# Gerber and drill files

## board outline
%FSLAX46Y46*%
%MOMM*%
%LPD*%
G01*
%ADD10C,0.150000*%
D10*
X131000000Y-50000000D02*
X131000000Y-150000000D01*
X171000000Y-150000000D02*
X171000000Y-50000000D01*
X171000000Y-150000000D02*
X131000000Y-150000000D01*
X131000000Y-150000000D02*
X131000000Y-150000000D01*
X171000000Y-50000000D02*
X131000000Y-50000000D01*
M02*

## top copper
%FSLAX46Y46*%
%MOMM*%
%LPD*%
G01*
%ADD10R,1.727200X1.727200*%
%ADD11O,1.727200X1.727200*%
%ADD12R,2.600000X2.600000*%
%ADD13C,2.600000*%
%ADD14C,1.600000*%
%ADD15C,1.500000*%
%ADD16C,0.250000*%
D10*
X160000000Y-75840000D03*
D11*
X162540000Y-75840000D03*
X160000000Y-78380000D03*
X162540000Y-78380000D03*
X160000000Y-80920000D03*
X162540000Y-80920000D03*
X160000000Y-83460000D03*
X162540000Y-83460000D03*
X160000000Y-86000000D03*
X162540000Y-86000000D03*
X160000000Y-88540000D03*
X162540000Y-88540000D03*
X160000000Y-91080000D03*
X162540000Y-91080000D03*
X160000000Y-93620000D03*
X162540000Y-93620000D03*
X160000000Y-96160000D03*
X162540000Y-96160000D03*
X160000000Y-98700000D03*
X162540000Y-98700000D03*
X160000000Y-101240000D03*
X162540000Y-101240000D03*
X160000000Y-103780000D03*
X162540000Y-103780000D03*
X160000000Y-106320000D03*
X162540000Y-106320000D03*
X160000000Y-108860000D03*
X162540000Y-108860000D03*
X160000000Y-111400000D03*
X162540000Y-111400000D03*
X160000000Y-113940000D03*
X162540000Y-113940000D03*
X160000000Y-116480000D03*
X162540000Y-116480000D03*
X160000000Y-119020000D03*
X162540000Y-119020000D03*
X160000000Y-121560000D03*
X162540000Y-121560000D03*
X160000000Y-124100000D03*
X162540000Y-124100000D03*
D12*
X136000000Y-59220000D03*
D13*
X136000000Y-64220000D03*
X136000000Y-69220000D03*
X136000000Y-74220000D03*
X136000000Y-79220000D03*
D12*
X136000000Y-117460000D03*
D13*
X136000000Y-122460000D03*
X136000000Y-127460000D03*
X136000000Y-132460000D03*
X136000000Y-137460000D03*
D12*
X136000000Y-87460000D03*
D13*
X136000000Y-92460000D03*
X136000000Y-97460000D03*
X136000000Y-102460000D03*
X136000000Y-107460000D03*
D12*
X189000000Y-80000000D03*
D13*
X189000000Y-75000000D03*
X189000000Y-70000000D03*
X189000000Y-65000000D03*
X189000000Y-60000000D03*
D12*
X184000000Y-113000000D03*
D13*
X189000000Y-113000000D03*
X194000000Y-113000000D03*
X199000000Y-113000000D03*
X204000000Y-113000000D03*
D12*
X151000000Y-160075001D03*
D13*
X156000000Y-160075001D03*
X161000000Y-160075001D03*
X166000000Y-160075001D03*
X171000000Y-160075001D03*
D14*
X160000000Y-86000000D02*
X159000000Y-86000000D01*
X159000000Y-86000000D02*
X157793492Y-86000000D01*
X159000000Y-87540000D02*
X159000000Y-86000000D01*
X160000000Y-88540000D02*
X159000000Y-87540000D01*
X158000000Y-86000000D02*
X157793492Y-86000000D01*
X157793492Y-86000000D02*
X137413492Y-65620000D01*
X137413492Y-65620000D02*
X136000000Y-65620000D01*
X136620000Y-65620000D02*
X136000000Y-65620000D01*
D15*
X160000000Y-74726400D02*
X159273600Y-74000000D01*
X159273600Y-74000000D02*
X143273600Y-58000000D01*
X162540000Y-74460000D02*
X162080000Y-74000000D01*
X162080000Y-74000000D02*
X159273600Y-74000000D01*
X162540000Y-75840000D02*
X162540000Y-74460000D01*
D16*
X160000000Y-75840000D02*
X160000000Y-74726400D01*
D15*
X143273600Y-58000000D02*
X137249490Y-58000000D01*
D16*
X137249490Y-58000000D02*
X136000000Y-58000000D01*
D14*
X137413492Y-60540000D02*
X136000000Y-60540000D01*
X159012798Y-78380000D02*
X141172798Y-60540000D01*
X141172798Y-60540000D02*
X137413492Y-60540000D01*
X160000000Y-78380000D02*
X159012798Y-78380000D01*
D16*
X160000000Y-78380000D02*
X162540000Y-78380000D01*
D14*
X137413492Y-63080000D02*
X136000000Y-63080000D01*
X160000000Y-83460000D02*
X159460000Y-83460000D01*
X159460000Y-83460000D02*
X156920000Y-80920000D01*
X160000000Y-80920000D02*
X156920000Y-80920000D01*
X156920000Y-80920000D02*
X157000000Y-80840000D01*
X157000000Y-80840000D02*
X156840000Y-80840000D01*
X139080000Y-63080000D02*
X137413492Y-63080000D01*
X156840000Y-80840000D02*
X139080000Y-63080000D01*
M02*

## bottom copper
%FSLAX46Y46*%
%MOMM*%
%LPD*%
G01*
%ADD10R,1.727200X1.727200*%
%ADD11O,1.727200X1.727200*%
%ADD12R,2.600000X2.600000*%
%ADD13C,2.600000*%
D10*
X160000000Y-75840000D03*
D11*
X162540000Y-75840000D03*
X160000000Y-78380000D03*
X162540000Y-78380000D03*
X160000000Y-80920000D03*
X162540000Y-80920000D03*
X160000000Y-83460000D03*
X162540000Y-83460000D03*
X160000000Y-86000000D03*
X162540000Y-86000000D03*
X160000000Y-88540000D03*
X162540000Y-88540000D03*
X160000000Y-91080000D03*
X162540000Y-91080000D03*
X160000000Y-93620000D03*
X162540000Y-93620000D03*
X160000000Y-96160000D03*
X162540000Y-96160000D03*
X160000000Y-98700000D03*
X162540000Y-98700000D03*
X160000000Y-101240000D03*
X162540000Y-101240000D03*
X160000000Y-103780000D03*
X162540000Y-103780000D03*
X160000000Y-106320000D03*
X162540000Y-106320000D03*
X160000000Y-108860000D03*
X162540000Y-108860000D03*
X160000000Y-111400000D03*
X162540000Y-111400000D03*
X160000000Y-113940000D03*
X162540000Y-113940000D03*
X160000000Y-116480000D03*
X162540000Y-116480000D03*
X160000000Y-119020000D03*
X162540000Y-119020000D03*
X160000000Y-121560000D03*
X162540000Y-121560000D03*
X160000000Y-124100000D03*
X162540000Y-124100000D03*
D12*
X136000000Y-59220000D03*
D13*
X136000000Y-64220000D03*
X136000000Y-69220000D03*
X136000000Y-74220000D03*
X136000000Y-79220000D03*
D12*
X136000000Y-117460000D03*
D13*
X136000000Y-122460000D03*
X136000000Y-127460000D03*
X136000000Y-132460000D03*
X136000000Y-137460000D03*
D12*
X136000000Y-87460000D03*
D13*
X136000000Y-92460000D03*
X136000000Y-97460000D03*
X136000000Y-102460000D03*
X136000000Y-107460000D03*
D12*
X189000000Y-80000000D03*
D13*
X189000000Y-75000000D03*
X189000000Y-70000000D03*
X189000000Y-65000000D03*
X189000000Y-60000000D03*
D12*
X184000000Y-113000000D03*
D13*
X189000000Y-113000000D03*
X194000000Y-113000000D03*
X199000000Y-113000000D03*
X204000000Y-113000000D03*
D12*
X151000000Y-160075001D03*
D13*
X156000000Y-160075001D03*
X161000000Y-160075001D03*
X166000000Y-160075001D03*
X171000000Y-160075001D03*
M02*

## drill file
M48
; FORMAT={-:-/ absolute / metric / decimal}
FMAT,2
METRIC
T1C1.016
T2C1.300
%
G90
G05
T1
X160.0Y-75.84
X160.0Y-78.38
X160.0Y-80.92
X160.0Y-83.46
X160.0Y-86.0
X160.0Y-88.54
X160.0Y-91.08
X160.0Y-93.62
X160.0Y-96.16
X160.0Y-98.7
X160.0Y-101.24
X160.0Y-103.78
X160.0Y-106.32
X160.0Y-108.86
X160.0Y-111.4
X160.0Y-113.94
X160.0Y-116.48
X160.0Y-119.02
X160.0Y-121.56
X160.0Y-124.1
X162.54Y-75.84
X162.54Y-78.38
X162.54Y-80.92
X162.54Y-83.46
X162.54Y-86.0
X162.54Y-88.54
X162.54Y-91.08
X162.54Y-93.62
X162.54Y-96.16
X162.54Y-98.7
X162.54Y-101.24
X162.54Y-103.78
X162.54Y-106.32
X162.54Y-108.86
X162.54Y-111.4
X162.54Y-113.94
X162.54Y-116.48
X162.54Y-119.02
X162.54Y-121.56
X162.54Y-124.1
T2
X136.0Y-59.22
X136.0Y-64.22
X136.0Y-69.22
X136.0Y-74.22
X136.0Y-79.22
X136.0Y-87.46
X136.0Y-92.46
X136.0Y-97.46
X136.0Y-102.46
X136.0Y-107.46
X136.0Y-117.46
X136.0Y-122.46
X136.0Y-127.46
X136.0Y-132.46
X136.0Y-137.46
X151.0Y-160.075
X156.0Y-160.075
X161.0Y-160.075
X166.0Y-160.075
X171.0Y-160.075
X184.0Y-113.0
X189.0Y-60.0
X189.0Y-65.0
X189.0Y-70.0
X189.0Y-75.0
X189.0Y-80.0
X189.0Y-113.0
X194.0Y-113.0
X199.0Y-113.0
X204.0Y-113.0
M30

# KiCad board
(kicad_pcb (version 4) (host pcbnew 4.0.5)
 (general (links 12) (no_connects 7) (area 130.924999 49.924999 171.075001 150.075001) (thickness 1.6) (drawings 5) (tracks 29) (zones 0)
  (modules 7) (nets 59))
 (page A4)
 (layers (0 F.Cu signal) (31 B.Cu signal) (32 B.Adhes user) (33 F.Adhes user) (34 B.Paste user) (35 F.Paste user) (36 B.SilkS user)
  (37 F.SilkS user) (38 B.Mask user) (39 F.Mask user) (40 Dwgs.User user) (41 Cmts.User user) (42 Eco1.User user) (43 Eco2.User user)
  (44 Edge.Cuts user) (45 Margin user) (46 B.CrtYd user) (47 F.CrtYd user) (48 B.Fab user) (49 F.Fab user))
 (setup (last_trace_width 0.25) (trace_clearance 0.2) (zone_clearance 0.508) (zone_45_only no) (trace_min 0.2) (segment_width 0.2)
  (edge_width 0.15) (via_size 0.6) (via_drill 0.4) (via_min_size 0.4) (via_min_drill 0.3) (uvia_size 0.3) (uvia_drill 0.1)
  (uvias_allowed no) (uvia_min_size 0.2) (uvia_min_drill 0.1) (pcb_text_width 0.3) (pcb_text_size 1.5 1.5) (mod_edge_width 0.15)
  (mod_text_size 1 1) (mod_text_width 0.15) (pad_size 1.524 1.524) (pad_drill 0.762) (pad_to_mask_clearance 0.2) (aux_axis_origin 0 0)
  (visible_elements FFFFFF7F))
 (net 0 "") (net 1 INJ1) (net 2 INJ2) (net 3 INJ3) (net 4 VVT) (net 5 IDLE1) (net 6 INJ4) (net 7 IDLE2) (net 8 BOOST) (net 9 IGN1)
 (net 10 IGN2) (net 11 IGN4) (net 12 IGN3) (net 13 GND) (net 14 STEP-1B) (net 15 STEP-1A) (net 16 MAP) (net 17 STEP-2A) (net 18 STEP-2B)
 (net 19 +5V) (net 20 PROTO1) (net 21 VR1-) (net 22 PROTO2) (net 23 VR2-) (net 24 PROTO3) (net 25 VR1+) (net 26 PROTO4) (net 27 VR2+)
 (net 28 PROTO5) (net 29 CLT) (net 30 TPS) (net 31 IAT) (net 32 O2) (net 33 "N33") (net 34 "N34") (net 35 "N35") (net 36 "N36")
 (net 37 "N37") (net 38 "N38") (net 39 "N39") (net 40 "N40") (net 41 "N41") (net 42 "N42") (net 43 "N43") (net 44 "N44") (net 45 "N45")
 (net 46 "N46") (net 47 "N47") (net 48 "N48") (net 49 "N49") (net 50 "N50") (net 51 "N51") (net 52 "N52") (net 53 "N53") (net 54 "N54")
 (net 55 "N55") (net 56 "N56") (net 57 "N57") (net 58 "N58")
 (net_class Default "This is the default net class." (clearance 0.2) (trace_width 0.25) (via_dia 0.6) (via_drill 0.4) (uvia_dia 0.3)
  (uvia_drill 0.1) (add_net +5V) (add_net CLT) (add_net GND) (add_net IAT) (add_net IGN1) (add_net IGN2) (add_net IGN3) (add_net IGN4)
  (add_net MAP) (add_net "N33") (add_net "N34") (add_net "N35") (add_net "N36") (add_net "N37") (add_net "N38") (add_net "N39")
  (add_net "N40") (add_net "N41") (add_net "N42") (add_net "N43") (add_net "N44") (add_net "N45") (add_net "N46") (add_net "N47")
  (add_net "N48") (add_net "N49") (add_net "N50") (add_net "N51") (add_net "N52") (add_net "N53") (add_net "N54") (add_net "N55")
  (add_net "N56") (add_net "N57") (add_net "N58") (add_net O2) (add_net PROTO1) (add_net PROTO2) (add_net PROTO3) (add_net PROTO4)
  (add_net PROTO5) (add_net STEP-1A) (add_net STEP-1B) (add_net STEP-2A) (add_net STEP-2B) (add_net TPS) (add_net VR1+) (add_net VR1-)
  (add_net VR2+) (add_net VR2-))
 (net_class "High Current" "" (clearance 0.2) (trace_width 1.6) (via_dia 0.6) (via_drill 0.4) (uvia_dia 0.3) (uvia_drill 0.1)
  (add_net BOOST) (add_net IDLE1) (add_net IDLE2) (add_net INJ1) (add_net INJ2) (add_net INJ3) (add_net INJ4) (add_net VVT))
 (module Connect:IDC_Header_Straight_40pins (layer F.Cu) (at 160 75.84 270)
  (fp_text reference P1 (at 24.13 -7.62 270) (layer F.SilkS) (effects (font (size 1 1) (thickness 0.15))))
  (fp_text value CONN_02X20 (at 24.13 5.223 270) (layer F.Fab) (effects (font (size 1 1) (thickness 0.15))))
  (pad 1 thru_hole rect (at 0 0 270) (size 1.7272 1.7272) (drill 1.016) (layers *.Cu *.Mask) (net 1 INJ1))
  (pad 2 thru_hole oval (at 0 -2.54 270) (size 1.7272 1.7272) (drill 1.016) (layers *.Cu *.Mask) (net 1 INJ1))
  (pad 3 thru_hole oval (at 2.54 0 270) (size 1.7272 1.7272) (drill 1.016) (layers *.Cu *.Mask) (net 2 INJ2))
  (pad 4 thru_hole oval (at 2.54 -2.54 270) (size 1.7272 1.7272) (drill 1.016) (layers *.Cu *.Mask) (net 2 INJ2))
  (pad 5 thru_hole oval (at 5.08 0 270) (size 1.7272 1.7272) (drill 1.016) (layers *.Cu *.Mask) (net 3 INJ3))
  (pad 6 thru_hole oval (at 5.08 -2.54 270) (size 1.7272 1.7272) (drill 1.016) (layers *.Cu *.Mask) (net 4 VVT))
  (pad 7 thru_hole oval (at 7.62 0 270) (size 1.7272 1.7272) (drill 1.016) (layers *.Cu *.Mask) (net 3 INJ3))
  (pad 8 thru_hole oval (at 7.62 -2.54 270) (size 1.7272 1.7272) (drill 1.016) (layers *.Cu *.Mask) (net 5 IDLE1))
  (pad 9 thru_hole oval (at 10.16 0 270) (size 1.7272 1.7272) (drill 1.016) (layers *.Cu *.Mask) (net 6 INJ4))
  (pad 10 thru_hole oval (at 10.16 -2.54 270) (size 1.7272 1.7272) (drill 1.016) (layers *.Cu *.Mask) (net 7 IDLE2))
  (pad 11 thru_hole oval (at 12.7 0 270) (size 1.7272 1.7272) (drill 1.016) (layers *.Cu *.Mask) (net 6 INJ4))
  (pad 12 thru_hole oval (at 12.7 -2.54 270) (size 1.7272 1.7272) (drill 1.016) (layers *.Cu *.Mask) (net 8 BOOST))
  (pad 13 thru_hole oval (at 15.24 0 270) (size 1.7272 1.7272) (drill 1.016) (layers *.Cu *.Mask) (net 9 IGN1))
  (pad 14 thru_hole oval (at 15.24 -2.54 270) (size 1.7272 1.7272) (drill 1.016) (layers *.Cu *.Mask) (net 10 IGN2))
  (pad 15 thru_hole oval (at 17.78 0 270) (size 1.7272 1.7272) (drill 1.016) (layers *.Cu *.Mask) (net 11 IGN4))
  (pad 16 thru_hole oval (at 17.78 -2.54 270) (size 1.7272 1.7272) (drill 1.016) (layers *.Cu *.Mask) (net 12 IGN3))
  (pad 17 thru_hole oval (at 20.32 0 270) (size 1.7272 1.7272) (drill 1.016) (layers *.Cu *.Mask) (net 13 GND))
  (pad 18 thru_hole oval (at 20.32 -2.54 270) (size 1.7272 1.7272) (drill 1.016) (layers *.Cu *.Mask) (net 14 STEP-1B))
  (pad 19 thru_hole oval (at 22.86 0 270) (size 1.7272 1.7272) (drill 1.016) (layers *.Cu *.Mask) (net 13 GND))
  (pad 20 thru_hole oval (at 22.86 -2.54 270) (size 1.7272 1.7272) (drill 1.016) (layers *.Cu *.Mask) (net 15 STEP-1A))
  (pad 21 thru_hole oval (at 25.4 0 270) (size 1.7272 1.7272) (drill 1.016) (layers *.Cu *.Mask) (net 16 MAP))
  (pad 22 thru_hole oval (at 25.4 -2.54 270) (size 1.7272 1.7272) (drill 1.016) (layers *.Cu *.Mask) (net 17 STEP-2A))
  (pad 23 thru_hole oval (at 27.94 0 270) (size 1.7272 1.7272) (drill 1.016) (layers *.Cu *.Mask) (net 13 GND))
  (pad 24 thru_hole oval (at 27.94 -2.54 270) (size 1.7272 1.7272) (drill 1.016) (layers *.Cu *.Mask) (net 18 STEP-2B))
  (pad 25 thru_hole oval (at 30.48 0 270) (size 1.7272 1.7272) (drill 1.016) (layers *.Cu *.Mask) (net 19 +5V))
  (pad 26 thru_hole oval (at 30.48 -2.54 270) (size 1.7272 1.7272) (drill 1.016) (layers *.Cu *.Mask) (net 19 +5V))
  (pad 27 thru_hole oval (at 33.02 0 270) (size 1.7272 1.7272) (drill 1.016) (layers *.Cu *.Mask) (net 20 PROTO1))
  (pad 28 thru_hole oval (at 33.02 -2.54 270) (size 1.7272 1.7272) (drill 1.016) (layers *.Cu *.Mask) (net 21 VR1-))
  (pad 29 thru_hole oval (at 35.56 0 270) (size 1.7272 1.7272) (drill 1.016) (layers *.Cu *.Mask) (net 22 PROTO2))
  (pad 30 thru_hole oval (at 35.56 -2.54 270) (size 1.7272 1.7272) (drill 1.016) (layers *.Cu *.Mask) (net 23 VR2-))
  (pad 31 thru_hole oval (at 38.1 0 270) (size 1.7272 1.7272) (drill 1.016) (layers *.Cu *.Mask) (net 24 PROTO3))
  (pad 32 thru_hole oval (at 38.1 -2.54 270) (size 1.7272 1.7272) (drill 1.016) (layers *.Cu *.Mask) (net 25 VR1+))
  (pad 33 thru_hole oval (at 40.64 0 270) (size 1.7272 1.7272) (drill 1.016) (layers *.Cu *.Mask) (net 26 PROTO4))
  (pad 34 thru_hole oval (at 40.64 -2.54 270) (size 1.7272 1.7272) (drill 1.016) (layers *.Cu *.Mask) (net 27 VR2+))
  (pad 35 thru_hole oval (at 43.18 0 270) (size 1.7272 1.7272) (drill 1.016) (layers *.Cu *.Mask) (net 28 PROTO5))
  (pad 36 thru_hole oval (at 43.18 -2.54 270) (size 1.7272 1.7272) (drill 1.016) (layers *.Cu *.Mask) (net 13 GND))
  (pad 37 thru_hole oval (at 45.72 0 270) (size 1.7272 1.7272) (drill 1.016) (layers *.Cu *.Mask) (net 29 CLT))
  (pad 38 thru_hole oval (at 45.72 -2.54 270) (size 1.7272 1.7272) (drill 1.016) (layers *.Cu *.Mask) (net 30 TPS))
  (pad 39 thru_hole oval (at 48.26 0 270) (size 1.7272 1.7272) (drill 1.016) (layers *.Cu *.Mask) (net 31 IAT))
  (pad 40 thru_hole oval (at 48.26 -2.54 270) (size 1.7272 1.7272) (drill 1.016) (layers *.Cu *.Mask) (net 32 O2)))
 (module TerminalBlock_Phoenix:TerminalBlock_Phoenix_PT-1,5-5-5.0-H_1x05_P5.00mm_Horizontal (layer F.Cu) (at 136 59.22 270)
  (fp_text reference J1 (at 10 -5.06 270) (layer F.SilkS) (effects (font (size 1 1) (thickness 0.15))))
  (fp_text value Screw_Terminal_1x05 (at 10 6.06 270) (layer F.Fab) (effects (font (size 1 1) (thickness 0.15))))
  (pad 1 thru_hole rect (at 0 0 270) (size 2.6 2.6) (drill 1.3) (layers *.Cu *.Mask) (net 1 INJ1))
  (pad 2 thru_hole circle (at 5 0 270) (size 2.6 2.6) (drill 1.3) (layers *.Cu *.Mask) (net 2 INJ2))
  (pad 3 thru_hole circle (at 10 0 270) (size 2.6 2.6) (drill 1.3) (layers *.Cu *.Mask) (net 3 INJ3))
  (pad 4 thru_hole circle (at 15 0 270) (size 2.6 2.6) (drill 1.3) (layers *.Cu *.Mask) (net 6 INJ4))
  (pad 5 thru_hole circle (at 20 0 270) (size 2.6 2.6) (drill 1.3) (layers *.Cu *.Mask) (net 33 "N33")))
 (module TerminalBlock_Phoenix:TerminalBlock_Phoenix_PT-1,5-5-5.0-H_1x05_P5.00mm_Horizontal (layer F.Cu) (at 136 117.46 270)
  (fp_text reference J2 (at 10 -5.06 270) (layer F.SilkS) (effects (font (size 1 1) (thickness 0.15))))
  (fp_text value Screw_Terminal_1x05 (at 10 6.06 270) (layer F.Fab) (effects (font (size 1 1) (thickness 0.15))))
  (pad 1 thru_hole rect (at 0 0 270) (size 2.6 2.6) (drill 1.3) (layers *.Cu *.Mask) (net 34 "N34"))
  (pad 2 thru_hole circle (at 5 0 270) (size 2.6 2.6) (drill 1.3) (layers *.Cu *.Mask) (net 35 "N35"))
  (pad 3 thru_hole circle (at 10 0 270) (size 2.6 2.6) (drill 1.3) (layers *.Cu *.Mask) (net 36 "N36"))
  (pad 4 thru_hole circle (at 15 0 270) (size 2.6 2.6) (drill 1.3) (layers *.Cu *.Mask) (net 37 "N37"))
  (pad 5 thru_hole circle (at 20 0 270) (size 2.6 2.6) (drill 1.3) (layers *.Cu *.Mask) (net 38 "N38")))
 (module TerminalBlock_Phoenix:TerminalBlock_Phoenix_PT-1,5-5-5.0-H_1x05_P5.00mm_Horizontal (layer F.Cu) (at 136 87.46 270)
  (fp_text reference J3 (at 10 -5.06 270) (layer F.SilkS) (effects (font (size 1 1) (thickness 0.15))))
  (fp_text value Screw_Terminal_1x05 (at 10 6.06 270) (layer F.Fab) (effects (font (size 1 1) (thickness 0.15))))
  (pad 1 thru_hole rect (at 0 0 270) (size 2.6 2.6) (drill 1.3) (layers *.Cu *.Mask) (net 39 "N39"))
  (pad 2 thru_hole circle (at 5 0 270) (size 2.6 2.6) (drill 1.3) (layers *.Cu *.Mask) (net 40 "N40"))
  (pad 3 thru_hole circle (at 10 0 270) (size 2.6 2.6) (drill 1.3) (layers *.Cu *.Mask) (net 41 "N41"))
  (pad 4 thru_hole circle (at 15 0 270) (size 2.6 2.6) (drill 1.3) (layers *.Cu *.Mask) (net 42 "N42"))
  (pad 5 thru_hole circle (at 20 0 270) (size 2.6 2.6) (drill 1.3) (layers *.Cu *.Mask) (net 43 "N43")))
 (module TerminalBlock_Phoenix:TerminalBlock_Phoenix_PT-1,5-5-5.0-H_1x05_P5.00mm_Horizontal (layer F.Cu) (at 189 80 90)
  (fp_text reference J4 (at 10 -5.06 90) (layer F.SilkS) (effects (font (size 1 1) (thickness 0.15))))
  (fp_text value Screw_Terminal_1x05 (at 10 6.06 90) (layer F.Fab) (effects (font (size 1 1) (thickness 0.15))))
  (pad 1 thru_hole rect (at 0 0 90) (size 2.6 2.6) (drill 1.3) (layers *.Cu *.Mask) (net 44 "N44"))
  (pad 2 thru_hole circle (at 5 0 90) (size 2.6 2.6) (drill 1.3) (layers *.Cu *.Mask) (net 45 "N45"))
  (pad 3 thru_hole circle (at 10 0 90) (size 2.6 2.6) (drill 1.3) (layers *.Cu *.Mask) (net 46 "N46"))
  (pad 4 thru_hole circle (at 15 0 90) (size 2.6 2.6) (drill 1.3) (layers *.Cu *.Mask) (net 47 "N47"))
  (pad 5 thru_hole circle (at 20 0 90) (size 2.6 2.6) (drill 1.3) (layers *.Cu *.Mask) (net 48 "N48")))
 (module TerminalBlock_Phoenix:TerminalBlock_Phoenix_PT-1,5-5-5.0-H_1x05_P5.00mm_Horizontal (layer F.Cu) (at 184 113)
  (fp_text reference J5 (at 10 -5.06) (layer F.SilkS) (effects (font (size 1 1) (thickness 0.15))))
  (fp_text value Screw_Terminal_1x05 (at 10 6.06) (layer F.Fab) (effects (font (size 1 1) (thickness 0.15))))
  (pad 1 thru_hole rect (at 0 0) (size 2.6 2.6) (drill 1.3) (layers *.Cu *.Mask) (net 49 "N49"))
  (pad 2 thru_hole circle (at 5 0) (size 2.6 2.6) (drill 1.3) (layers *.Cu *.Mask) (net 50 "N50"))
  (pad 3 thru_hole circle (at 10 0) (size 2.6 2.6) (drill 1.3) (layers *.Cu *.Mask) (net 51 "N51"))
  (pad 4 thru_hole circle (at 15 0) (size 2.6 2.6) (drill 1.3) (layers *.Cu *.Mask) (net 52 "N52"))
  (pad 5 thru_hole circle (at 20 0) (size 2.6 2.6) (drill 1.3) (layers *.Cu *.Mask) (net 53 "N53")))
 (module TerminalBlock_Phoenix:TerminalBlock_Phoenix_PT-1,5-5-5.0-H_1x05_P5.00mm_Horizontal (layer F.Cu) (at 151 160.075001)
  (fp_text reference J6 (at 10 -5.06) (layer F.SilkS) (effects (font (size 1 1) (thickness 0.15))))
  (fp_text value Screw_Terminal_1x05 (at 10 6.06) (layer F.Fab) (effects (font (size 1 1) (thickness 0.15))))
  (pad 1 thru_hole rect (at 0 0) (size 2.6 2.6) (drill 1.3) (layers *.Cu *.Mask) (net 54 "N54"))
  (pad 2 thru_hole circle (at 5 0) (size 2.6 2.6) (drill 1.3) (layers *.Cu *.Mask) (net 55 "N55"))
  (pad 3 thru_hole circle (at 10 0) (size 2.6 2.6) (drill 1.3) (layers *.Cu *.Mask) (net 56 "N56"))
  (pad 4 thru_hole circle (at 15 0) (size 2.6 2.6) (drill 1.3) (layers *.Cu *.Mask) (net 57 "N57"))
  (pad 5 thru_hole circle (at 20 0) (size 2.6 2.6) (drill 1.3) (layers *.Cu *.Mask) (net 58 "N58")))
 (gr_line (start 131 50) (end 131 150) (layer Edge.Cuts) (width 0.15))
 (gr_line (start 171 150) (end 171 50) (layer Edge.Cuts) (width 0.15))
 (gr_line (start 171 150) (end 131 150) (layer Edge.Cuts) (width 0.15))
 (gr_line (start 131 150) (end 131 150) (layer Edge.Cuts) (width 0.15))
 (gr_line (start 171 50) (end 131 50) (layer Edge.Cuts) (width 0.15))
 (segment (start 160 86) (end 159 86) (width 1.6) (layer F.Cu) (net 6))
 (segment (start 159 86) (end 157.793492 86) (width 1.6) (layer F.Cu) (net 6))
 (segment (start 159 87.54) (end 159 86) (width 1.6) (layer F.Cu) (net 6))
 (segment (start 160 88.54) (end 159 87.54) (width 1.6) (layer F.Cu) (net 6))
 (segment (start 158 86) (end 157.793492 86) (width 1.6) (layer F.Cu) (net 6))
 (segment (start 157.793492 86) (end 137.413492 65.62) (width 1.6) (layer F.Cu) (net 6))
 (segment (start 137.413492 65.62) (end 136 65.62) (width 1.6) (layer F.Cu) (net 6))
 (segment (start 136.62 65.62) (end 136 65.62) (width 1.6) (layer F.Cu) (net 6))
 (segment (start 160 74.7264) (end 159.2736 74) (width 1.5) (layer F.Cu) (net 1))
 (segment (start 159.2736 74) (end 143.2736 58) (width 1.5) (layer F.Cu) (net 1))
 (segment (start 162.54 74.46) (end 162.08 74) (width 1.5) (layer F.Cu) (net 1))
 (segment (start 162.08 74) (end 159.2736 74) (width 1.5) (layer F.Cu) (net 1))
 (segment (start 162.54 75.84) (end 162.54 74.46) (width 1.5) (layer F.Cu) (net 1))
 (segment (start 160 75.84) (end 160 74.7264) (width 0.25) (layer F.Cu) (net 1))
 (segment (start 143.2736 58) (end 137.24949 58) (width 1.5) (layer F.Cu) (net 1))
 (segment (start 137.24949 58) (end 136 58) (width 0.25) (layer F.Cu) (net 1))
 (segment (start 137.413492 60.54) (end 136 60.54) (width 1.6) (layer F.Cu) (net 2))
 (segment (start 159.012798 78.38) (end 141.172798 60.54) (width 1.6) (layer F.Cu) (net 2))
 (segment (start 141.172798 60.54) (end 137.413492 60.54) (width 1.6) (layer F.Cu) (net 2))
 (segment (start 160 78.38) (end 159.012798 78.38) (width 1.6) (layer F.Cu) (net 2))
 (segment (start 160 78.38) (end 162.54 78.38) (width 0.25) (layer F.Cu) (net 2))
 (segment (start 137.413492 63.08) (end 136 63.08) (width 1.6) (layer F.Cu) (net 2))
 (segment (start 160 83.46) (end 159.46 83.46) (width 1.6) (layer F.Cu) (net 3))
 (segment (start 159.46 83.46) (end 156.92 80.92) (width 1.6) (layer F.Cu) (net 3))
 (segment (start 160 80.92) (end 156.92 80.92) (width 1.6) (layer F.Cu) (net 3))
 (segment (start 156.92 80.92) (end 157 80.84) (width 1.6) (layer F.Cu) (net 3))
 (segment (start 157 80.84) (end 156.84 80.84) (width 1.6) (layer F.Cu) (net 3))
 (segment (start 139.08 63.08) (end 137.413492 63.08) (width 1.6) (layer F.Cu) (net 3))
 (segment (start 156.84 80.84) (end 139.08 63.08) (width 1.6) (layer F.Cu) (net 3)))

